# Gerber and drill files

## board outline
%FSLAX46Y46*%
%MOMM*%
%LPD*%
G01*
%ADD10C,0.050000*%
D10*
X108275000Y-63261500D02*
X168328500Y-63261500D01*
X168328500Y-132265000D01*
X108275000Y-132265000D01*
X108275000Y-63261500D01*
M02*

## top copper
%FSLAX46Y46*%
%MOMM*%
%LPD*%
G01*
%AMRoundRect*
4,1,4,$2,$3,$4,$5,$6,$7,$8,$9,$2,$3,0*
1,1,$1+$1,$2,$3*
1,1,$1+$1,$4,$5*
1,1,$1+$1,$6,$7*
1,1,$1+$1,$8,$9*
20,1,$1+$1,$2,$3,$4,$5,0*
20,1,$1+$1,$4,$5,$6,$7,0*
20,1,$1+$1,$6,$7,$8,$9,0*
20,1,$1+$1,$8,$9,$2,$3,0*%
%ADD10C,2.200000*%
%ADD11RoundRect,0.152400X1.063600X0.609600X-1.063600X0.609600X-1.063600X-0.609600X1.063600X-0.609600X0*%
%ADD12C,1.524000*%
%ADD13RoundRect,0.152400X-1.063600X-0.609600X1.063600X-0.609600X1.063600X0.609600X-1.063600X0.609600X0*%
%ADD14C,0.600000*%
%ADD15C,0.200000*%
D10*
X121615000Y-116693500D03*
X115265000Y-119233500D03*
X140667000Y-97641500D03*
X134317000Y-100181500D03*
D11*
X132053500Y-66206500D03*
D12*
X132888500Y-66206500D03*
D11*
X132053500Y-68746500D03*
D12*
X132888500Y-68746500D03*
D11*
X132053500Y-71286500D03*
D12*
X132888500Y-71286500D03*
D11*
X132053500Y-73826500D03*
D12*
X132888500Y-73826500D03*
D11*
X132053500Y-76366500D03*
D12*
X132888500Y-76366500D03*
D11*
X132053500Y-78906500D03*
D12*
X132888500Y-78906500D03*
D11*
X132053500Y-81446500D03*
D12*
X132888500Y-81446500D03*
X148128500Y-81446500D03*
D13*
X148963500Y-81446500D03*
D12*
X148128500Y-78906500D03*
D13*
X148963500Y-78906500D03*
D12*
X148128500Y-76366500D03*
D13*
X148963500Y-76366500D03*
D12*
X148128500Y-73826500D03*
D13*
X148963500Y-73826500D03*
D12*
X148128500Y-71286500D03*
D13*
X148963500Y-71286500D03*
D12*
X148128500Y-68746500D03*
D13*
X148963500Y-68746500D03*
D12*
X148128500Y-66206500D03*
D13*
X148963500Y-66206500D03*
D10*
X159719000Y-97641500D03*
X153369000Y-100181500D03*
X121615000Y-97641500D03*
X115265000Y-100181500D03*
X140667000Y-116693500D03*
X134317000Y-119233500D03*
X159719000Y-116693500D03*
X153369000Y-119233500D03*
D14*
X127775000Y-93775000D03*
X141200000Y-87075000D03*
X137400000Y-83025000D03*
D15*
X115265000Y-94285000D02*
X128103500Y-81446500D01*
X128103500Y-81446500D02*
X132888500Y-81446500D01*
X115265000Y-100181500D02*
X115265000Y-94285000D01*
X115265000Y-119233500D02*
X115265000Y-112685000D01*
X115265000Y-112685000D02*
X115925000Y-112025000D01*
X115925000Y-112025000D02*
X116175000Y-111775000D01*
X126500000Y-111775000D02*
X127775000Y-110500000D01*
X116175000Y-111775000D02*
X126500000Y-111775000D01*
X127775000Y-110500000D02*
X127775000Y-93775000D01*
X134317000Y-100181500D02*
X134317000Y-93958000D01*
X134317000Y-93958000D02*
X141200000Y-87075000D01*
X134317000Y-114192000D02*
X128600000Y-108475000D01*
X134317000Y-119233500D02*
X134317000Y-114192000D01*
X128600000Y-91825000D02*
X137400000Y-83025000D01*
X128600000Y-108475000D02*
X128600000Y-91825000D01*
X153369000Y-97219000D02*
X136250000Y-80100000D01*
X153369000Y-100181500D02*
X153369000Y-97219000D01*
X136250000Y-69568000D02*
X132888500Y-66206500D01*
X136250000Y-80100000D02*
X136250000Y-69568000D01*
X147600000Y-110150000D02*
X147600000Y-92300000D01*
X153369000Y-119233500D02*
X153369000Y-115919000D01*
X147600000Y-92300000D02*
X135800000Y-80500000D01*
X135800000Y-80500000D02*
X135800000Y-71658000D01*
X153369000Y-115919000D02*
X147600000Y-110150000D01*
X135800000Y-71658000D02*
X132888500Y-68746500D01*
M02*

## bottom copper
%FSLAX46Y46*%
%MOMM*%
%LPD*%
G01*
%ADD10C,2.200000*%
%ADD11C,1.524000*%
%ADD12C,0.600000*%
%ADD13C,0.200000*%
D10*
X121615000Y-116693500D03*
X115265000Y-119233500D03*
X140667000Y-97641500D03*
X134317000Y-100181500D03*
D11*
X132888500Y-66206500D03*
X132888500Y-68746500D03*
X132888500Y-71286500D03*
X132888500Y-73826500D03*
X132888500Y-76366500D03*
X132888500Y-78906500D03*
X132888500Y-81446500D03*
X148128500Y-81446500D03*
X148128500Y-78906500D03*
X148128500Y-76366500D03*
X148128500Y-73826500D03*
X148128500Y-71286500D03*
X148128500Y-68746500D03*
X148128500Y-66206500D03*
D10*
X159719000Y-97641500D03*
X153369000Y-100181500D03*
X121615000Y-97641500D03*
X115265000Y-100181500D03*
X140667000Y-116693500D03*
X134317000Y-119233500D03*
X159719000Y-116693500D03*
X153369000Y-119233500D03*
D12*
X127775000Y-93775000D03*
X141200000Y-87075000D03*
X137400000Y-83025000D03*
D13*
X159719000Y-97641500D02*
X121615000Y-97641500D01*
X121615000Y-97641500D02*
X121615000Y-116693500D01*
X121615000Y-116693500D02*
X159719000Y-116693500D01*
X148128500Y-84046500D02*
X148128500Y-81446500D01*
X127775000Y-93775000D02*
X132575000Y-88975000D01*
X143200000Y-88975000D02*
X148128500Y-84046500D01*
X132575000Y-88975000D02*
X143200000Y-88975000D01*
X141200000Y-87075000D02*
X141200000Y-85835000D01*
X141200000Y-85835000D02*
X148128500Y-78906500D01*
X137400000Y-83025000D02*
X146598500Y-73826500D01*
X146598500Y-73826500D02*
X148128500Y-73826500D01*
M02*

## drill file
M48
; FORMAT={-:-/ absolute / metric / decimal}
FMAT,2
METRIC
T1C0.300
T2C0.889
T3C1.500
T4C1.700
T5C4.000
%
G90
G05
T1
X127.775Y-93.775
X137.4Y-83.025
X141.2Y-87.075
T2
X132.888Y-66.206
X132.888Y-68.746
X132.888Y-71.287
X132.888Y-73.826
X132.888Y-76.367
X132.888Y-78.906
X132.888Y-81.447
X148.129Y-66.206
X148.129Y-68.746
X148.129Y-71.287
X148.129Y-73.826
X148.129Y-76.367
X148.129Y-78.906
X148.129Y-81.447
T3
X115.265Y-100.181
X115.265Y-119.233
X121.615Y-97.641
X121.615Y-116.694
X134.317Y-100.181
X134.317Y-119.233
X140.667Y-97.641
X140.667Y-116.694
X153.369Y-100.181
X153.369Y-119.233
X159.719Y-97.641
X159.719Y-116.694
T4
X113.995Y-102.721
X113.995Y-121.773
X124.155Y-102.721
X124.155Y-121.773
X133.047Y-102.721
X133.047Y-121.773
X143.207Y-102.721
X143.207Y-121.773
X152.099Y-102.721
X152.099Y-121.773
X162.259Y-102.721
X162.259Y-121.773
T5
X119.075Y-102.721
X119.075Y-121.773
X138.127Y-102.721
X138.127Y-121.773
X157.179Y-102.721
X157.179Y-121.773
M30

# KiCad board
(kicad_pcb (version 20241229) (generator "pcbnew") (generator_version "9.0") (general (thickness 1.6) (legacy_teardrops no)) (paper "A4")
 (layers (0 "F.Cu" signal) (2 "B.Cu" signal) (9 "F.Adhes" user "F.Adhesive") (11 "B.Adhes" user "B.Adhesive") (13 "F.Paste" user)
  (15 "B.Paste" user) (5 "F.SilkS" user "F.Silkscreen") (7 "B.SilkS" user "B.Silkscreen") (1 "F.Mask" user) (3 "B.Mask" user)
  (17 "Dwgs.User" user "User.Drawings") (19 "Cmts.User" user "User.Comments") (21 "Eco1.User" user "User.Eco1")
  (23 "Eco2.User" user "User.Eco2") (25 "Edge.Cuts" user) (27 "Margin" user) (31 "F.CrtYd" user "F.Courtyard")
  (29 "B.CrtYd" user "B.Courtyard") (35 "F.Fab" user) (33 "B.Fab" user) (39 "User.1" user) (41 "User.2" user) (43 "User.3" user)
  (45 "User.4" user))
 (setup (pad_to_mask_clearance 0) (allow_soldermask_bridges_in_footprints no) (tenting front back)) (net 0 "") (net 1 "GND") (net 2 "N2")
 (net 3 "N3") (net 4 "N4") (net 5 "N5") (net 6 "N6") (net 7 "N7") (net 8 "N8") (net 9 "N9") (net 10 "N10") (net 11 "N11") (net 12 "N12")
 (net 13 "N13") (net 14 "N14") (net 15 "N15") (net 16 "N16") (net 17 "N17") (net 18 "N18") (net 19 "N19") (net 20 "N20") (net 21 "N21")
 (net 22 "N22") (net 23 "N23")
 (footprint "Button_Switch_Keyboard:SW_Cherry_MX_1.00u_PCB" (layer "F.Cu") (at 121.615 116.6935)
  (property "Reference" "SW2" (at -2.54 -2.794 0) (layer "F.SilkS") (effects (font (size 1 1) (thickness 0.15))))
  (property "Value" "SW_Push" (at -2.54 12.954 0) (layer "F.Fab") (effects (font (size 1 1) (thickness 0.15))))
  (pad "" np_thru_hole circle (at -7.62 5.08) (size 1.7 1.7) (drill 1.7) (layers "*.Cu" "*.Mask"))
  (pad "" np_thru_hole circle (at -2.54 5.08) (size 4 4) (drill 4) (layers "*.Cu" "*.Mask"))
  (pad "" np_thru_hole circle (at 2.54 5.08) (size 1.7 1.7) (drill 1.7) (layers "*.Cu" "*.Mask"))
  (pad "1" thru_hole circle (at 0 0) (size 2.2 2.2) (drill 1.5) (layers "*.Cu" "*.Mask") (remove_unused_layers no) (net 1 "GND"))
  (pad "2" thru_hole circle (at -6.35 2.54) (size 2.2 2.2) (drill 1.5) (layers "*.Cu" "*.Mask") (remove_unused_layers no) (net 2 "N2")))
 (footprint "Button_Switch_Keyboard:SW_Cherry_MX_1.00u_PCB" (layer "F.Cu") (at 140.667 97.6415)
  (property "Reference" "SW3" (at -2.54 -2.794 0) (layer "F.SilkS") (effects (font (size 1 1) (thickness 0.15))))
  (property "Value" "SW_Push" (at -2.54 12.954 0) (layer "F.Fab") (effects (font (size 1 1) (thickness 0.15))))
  (pad "" np_thru_hole circle (at -7.62 5.08) (size 1.7 1.7) (drill 1.7) (layers "*.Cu" "*.Mask"))
  (pad "" np_thru_hole circle (at -2.54 5.08) (size 4 4) (drill 4) (layers "*.Cu" "*.Mask"))
  (pad "" np_thru_hole circle (at 2.54 5.08) (size 1.7 1.7) (drill 1.7) (layers "*.Cu" "*.Mask"))
  (pad "1" thru_hole circle (at 0 0) (size 2.2 2.2) (drill 1.5) (layers "*.Cu" "*.Mask") (remove_unused_layers no) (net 1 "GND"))
  (pad "2" thru_hole circle (at -6.35 2.54) (size 2.2 2.2) (drill 1.5) (layers "*.Cu" "*.Mask") (remove_unused_layers no) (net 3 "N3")))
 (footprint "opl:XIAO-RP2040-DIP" (layer "F.Cu") (at 140.5085 73.8265)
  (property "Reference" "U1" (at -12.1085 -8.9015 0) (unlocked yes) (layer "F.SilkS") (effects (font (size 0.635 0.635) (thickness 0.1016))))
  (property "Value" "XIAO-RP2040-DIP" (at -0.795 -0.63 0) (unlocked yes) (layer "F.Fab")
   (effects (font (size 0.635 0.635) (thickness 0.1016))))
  (pad "1" smd roundrect (at -8.455 -7.62 180) (size 2.432 1.524) (layers "F.Cu" "F.Mask") (roundrect_rratio 0.1) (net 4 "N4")
   (thermal_bridge_angle 45))
  (pad "1" thru_hole circle (at -7.62 -7.62 180) (size 1.524 1.524) (drill 0.889) (layers "*.Cu" "*.Mask") (remove_unused_layers no)
   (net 4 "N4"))
  (pad "2" smd roundrect (at -8.455 -5.08 180) (size 2.432 1.524) (layers "F.Cu" "F.Mask") (roundrect_rratio 0.1) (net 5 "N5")
   (thermal_bridge_angle 45))
  (pad "2" thru_hole circle (at -7.62 -5.08 180) (size 1.524 1.524) (drill 0.889) (layers "*.Cu" "*.Mask") (remove_unused_layers no)
   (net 5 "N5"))
  (pad "3" smd roundrect (at -8.455 -2.54 180) (size 2.432 1.524) (layers "F.Cu" "F.Mask") (roundrect_rratio 0.1) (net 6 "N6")
   (thermal_bridge_angle 45))
  (pad "3" thru_hole circle (at -7.62 -2.54 180) (size 1.524 1.524) (drill 0.889) (layers "*.Cu" "*.Mask") (remove_unused_layers no)
   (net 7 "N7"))
  (pad "4" smd roundrect (at -8.455 0 180) (size 2.432 1.524) (layers "F.Cu" "F.Mask") (roundrect_rratio 0.1) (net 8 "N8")
   (thermal_bridge_angle 45))
  (pad "4" thru_hole circle (at -7.62 0 180) (size 1.524 1.524) (drill 0.889) (layers "*.Cu" "*.Mask") (remove_unused_layers no)
   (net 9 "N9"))
  (pad "5" smd roundrect (at -8.455 2.54 180) (size 2.432 1.524) (layers "F.Cu" "F.Mask") (roundrect_rratio 0.1) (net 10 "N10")
   (thermal_bridge_angle 45))
  (pad "5" thru_hole circle (at -7.62 2.54 180) (size 1.524 1.524) (drill 0.889) (layers "*.Cu" "*.Mask") (remove_unused_layers no)
   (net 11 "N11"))
  (pad "6" smd roundrect (at -8.455 5.08 180) (size 2.432 1.524) (layers "F.Cu" "F.Mask") (roundrect_rratio 0.1) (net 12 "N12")
   (thermal_bridge_angle 45))
  (pad "6" thru_hole circle (at -7.62 5.08 180) (size 1.524 1.524) (drill 0.889) (layers "*.Cu" "*.Mask") (remove_unused_layers no)
   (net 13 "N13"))
  (pad "7" smd roundrect (at -8.455 7.62 180) (size 2.432 1.524) (layers "F.Cu" "F.Mask") (roundrect_rratio 0.1) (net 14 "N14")
   (thermal_bridge_angle 45))
  (pad "7" thru_hole circle (at -7.62 7.62 180) (size 1.524 1.524) (drill 0.889) (layers "*.Cu" "*.Mask") (remove_unused_layers no)
   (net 14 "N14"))
  (pad "8" thru_hole circle (at 7.62 7.62) (size 1.524 1.524) (drill 0.889) (layers "*.Cu" "*.Mask") (remove_unused_layers no) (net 2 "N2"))
  (pad "8" smd roundrect (at 8.455 7.62) (size 2.432 1.524) (layers "F.Cu" "F.Mask") (roundrect_rratio 0.1) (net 2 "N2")
   (thermal_bridge_angle 45))
  (pad "9" thru_hole circle (at 7.62 5.08) (size 1.524 1.524) (drill 0.889) (layers "*.Cu" "*.Mask") (remove_unused_layers no) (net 3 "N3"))
  (pad "9" smd roundrect (at 8.455 5.08) (size 2.432 1.524) (layers "F.Cu" "F.Mask") (roundrect_rratio 0.1) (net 3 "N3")
   (thermal_bridge_angle 45))
  (pad "10" thru_hole circle (at 7.62 2.54) (size 1.524 1.524) (drill 0.889) (layers "*.Cu" "*.Mask") (remove_unused_layers no)
   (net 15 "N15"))
  (pad "10" smd roundrect (at 8.455 2.54) (size 2.432 1.524) (layers "F.Cu" "F.Mask") (roundrect_rratio 0.1) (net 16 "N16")
   (thermal_bridge_angle 45))
  (pad "11" thru_hole circle (at 7.62 0) (size 1.524 1.524) (drill 0.889) (layers "*.Cu" "*.Mask") (remove_unused_layers no) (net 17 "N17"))
  (pad "11" smd roundrect (at 8.455 0) (size 2.432 1.524) (layers "F.Cu" "F.Mask") (roundrect_rratio 0.1) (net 17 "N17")
   (thermal_bridge_angle 45))
  (pad "12" thru_hole circle (at 7.62 -2.54) (size 1.524 1.524) (drill 0.889) (layers "*.Cu" "*.Mask") (remove_unused_layers no)
   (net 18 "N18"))
  (pad "12" smd roundrect (at 8.455 -2.54) (size 2.432 1.524) (layers "F.Cu" "F.Mask") (roundrect_rratio 0.1) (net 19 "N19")
   (thermal_bridge_angle 45))
  (pad "13" thru_hole circle (at 7.62 -5.08) (size 1.524 1.524) (drill 0.889) (layers "*.Cu" "*.Mask") (remove_unused_layers no)
   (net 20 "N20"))
  (pad "13" smd roundrect (at 8.455 -5.08) (size 2.432 1.524) (layers "F.Cu" "F.Mask") (roundrect_rratio 0.1) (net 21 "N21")
   (thermal_bridge_angle 45))
  (pad "14" thru_hole circle (at 7.62 -7.62) (size 1.524 1.524) (drill 0.889) (layers "*.Cu" "*.Mask") (remove_unused_layers no)
   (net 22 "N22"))
  (pad "14" smd roundrect (at 8.455 -7.62) (size 2.432 1.524) (layers "F.Cu" "F.Mask") (roundrect_rratio 0.1) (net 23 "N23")
   (thermal_bridge_angle 45)))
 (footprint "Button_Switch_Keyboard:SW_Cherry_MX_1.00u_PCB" (layer "F.Cu") (at 159.719 97.6415)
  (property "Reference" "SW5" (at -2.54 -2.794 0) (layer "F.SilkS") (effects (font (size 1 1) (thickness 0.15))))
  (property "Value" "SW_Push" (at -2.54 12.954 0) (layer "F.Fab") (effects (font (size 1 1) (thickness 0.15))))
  (pad "" np_thru_hole circle (at -7.62 5.08) (size 1.7 1.7) (drill 1.7) (layers "*.Cu" "*.Mask"))
  (pad "" np_thru_hole circle (at -2.54 5.08) (size 4 4) (drill 4) (layers "*.Cu" "*.Mask"))
  (pad "" np_thru_hole circle (at 2.54 5.08) (size 1.7 1.7) (drill 1.7) (layers "*.Cu" "*.Mask"))
  (pad "1" thru_hole circle (at 0 0) (size 2.2 2.2) (drill 1.5) (layers "*.Cu" "*.Mask") (remove_unused_layers no) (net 1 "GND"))
  (pad "2" thru_hole circle (at -6.35 2.54) (size 2.2 2.2) (drill 1.5) (layers "*.Cu" "*.Mask") (remove_unused_layers no) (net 4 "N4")))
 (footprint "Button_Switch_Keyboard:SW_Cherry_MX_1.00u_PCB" (layer "F.Cu") (at 121.615 97.6415)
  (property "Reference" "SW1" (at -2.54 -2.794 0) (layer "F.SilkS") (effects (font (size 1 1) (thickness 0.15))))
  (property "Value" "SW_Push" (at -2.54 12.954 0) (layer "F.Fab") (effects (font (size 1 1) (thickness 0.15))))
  (pad "" np_thru_hole circle (at -7.62 5.08) (size 1.7 1.7) (drill 1.7) (layers "*.Cu" "*.Mask"))
  (pad "" np_thru_hole circle (at -2.54 5.08) (size 4 4) (drill 4) (layers "*.Cu" "*.Mask"))
  (pad "" np_thru_hole circle (at 2.54 5.08) (size 1.7 1.7) (drill 1.7) (layers "*.Cu" "*.Mask"))
  (pad "1" thru_hole circle (at 0 0) (size 2.2 2.2) (drill 1.5) (layers "*.Cu" "*.Mask") (remove_unused_layers no) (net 1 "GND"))
  (pad "2" thru_hole circle (at -6.35 2.54) (size 2.2 2.2) (drill 1.5) (layers "*.Cu" "*.Mask") (remove_unused_layers no) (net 14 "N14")))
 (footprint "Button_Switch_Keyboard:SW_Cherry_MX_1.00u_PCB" (layer "F.Cu") (at 140.667 116.6935)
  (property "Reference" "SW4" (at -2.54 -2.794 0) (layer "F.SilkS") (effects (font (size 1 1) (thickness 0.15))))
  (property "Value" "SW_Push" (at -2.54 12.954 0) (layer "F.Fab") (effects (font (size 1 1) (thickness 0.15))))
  (pad "" np_thru_hole circle (at -7.62 5.08) (size 1.7 1.7) (drill 1.7) (layers "*.Cu" "*.Mask"))
  (pad "" np_thru_hole circle (at -2.54 5.08) (size 4 4) (drill 4) (layers "*.Cu" "*.Mask"))
  (pad "" np_thru_hole circle (at 2.54 5.08) (size 1.7 1.7) (drill 1.7) (layers "*.Cu" "*.Mask"))
  (pad "1" thru_hole circle (at 0 0) (size 2.2 2.2) (drill 1.5) (layers "*.Cu" "*.Mask") (remove_unused_layers no) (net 1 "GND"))
  (pad "2" thru_hole circle (at -6.35 2.54) (size 2.2 2.2) (drill 1.5) (layers "*.Cu" "*.Mask") (remove_unused_layers no) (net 17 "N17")))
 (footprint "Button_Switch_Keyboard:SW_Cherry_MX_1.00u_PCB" (layer "F.Cu") (at 159.719 116.6935)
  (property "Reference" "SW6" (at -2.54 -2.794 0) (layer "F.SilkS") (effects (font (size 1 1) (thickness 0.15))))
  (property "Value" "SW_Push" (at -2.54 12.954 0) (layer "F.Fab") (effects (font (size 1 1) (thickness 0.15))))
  (pad "" np_thru_hole circle (at -7.62 5.08) (size 1.7 1.7) (drill 1.7) (layers "*.Cu" "*.Mask"))
  (pad "" np_thru_hole circle (at -2.54 5.08) (size 4 4) (drill 4) (layers "*.Cu" "*.Mask"))
  (pad "" np_thru_hole circle (at 2.54 5.08) (size 1.7 1.7) (drill 1.7) (layers "*.Cu" "*.Mask"))
  (pad "1" thru_hole circle (at 0 0) (size 2.2 2.2) (drill 1.5) (layers "*.Cu" "*.Mask") (remove_unused_layers no) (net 1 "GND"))
  (pad "2" thru_hole circle (at -6.35 2.54) (size 2.2 2.2) (drill 1.5) (layers "*.Cu" "*.Mask") (remove_unused_layers no) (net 5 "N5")))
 (gr_rect (start 108.275 63.2615) (end 168.3285 132.265) (stroke (width 0.05) (type default)) (fill no) (layer "Edge.Cuts"))
 (segment (start 115.265 94.285) (end 128.1035 81.4465) (width 0.2) (layer "F.Cu") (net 14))
 (segment (start 128.1035 81.4465) (end 132.8885 81.4465) (width 0.2) (layer "F.Cu") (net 14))
 (segment (start 115.265 100.1815) (end 115.265 94.285) (width 0.2) (layer "F.Cu") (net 14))
 (segment (start 159.719 97.6415) (end 121.615 97.6415) (width 0.2) (layer "B.Cu") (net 1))
 (segment (start 121.615 97.6415) (end 121.615 116.6935) (width 0.2) (layer "B.Cu") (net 1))
 (segment (start 121.615 116.6935) (end 159.719 116.6935) (width 0.2) (layer "B.Cu") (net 1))
 (segment (start 115.265 119.2335) (end 115.265 112.685) (width 0.2) (layer "F.Cu") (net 2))
 (segment (start 115.265 112.685) (end 115.925 112.025) (width 0.2) (layer "F.Cu") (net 2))
 (segment (start 115.925 112.025) (end 116.175 111.775) (width 0.2) (layer "F.Cu") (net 2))
 (segment (start 126.5 111.775) (end 127.775 110.5) (width 0.2) (layer "F.Cu") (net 2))
 (segment (start 116.175 111.775) (end 126.5 111.775) (width 0.2) (layer "F.Cu") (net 2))
 (segment (start 127.775 110.5) (end 127.775 93.775) (width 0.2) (layer "F.Cu") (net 2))
 (via (at 127.775 93.775) (size 0.6) (drill 0.3) (layers "F.Cu" "B.Cu") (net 2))
 (segment (start 148.1285 84.0465) (end 148.1285 81.4465) (width 0.2) (layer "B.Cu") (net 2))
 (segment (start 127.775 93.775) (end 132.575 88.975) (width 0.2) (layer "B.Cu") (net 2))
 (segment (start 143.2 88.975) (end 148.1285 84.0465) (width 0.2) (layer "B.Cu") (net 2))
 (segment (start 132.575 88.975) (end 143.2 88.975) (width 0.2) (layer "B.Cu") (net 2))
 (segment (start 134.317 100.1815) (end 134.317 93.958) (width 0.2) (layer "F.Cu") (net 3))
 (segment (start 134.317 93.958) (end 141.2 87.075) (width 0.2) (layer "F.Cu") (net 3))
 (via (at 141.2 87.075) (size 0.6) (drill 0.3) (layers "F.Cu" "B.Cu") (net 3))
 (segment (start 141.2 87.075) (end 141.2 85.835) (width 0.2) (layer "B.Cu") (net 3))
 (segment (start 141.2 85.835) (end 148.1285 78.9065) (width 0.2) (layer "B.Cu") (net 3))
 (segment (start 134.317 114.192) (end 128.6 108.475) (width 0.2) (layer "F.Cu") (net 17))
 (segment (start 134.317 119.2335) (end 134.317 114.192) (width 0.2) (layer "F.Cu") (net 17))
 (segment (start 128.6 91.825) (end 137.4 83.025) (width 0.2) (layer "F.Cu") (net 17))
 (segment (start 128.6 108.475) (end 128.6 91.825) (width 0.2) (layer "F.Cu") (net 17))
 (via (at 137.4 83.025) (size 0.6) (drill 0.3) (layers "F.Cu" "B.Cu") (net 17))
 (segment (start 137.4 83.025) (end 146.5985 73.8265) (width 0.2) (layer "B.Cu") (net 17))
 (segment (start 146.5985 73.8265) (end 148.1285 73.8265) (width 0.2) (layer "B.Cu") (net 17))
 (segment (start 153.369 97.219) (end 136.25 80.1) (width 0.2) (layer "F.Cu") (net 4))
 (segment (start 153.369 100.1815) (end 153.369 97.219) (width 0.2) (layer "F.Cu") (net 4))
 (segment (start 136.25 69.568) (end 132.8885 66.2065) (width 0.2) (layer "F.Cu") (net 4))
 (segment (start 136.25 80.1) (end 136.25 69.568) (width 0.2) (layer "F.Cu") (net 4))
 (segment (start 147.6 110.15) (end 147.6 92.3) (width 0.2) (layer "F.Cu") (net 5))
 (segment (start 153.369 119.2335) (end 153.369 115.919) (width 0.2) (layer "F.Cu") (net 5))
 (segment (start 147.6 92.3) (end 135.8 80.5) (width 0.2) (layer "F.Cu") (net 5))
 (segment (start 135.8 80.5) (end 135.8 71.658) (width 0.2) (layer "F.Cu") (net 5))
 (segment (start 153.369 115.919) (end 147.6 110.15) (width 0.2) (layer "F.Cu") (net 5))
 (segment (start 135.8 71.658) (end 132.8885 68.7465) (width 0.2) (layer "F.Cu") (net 5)))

